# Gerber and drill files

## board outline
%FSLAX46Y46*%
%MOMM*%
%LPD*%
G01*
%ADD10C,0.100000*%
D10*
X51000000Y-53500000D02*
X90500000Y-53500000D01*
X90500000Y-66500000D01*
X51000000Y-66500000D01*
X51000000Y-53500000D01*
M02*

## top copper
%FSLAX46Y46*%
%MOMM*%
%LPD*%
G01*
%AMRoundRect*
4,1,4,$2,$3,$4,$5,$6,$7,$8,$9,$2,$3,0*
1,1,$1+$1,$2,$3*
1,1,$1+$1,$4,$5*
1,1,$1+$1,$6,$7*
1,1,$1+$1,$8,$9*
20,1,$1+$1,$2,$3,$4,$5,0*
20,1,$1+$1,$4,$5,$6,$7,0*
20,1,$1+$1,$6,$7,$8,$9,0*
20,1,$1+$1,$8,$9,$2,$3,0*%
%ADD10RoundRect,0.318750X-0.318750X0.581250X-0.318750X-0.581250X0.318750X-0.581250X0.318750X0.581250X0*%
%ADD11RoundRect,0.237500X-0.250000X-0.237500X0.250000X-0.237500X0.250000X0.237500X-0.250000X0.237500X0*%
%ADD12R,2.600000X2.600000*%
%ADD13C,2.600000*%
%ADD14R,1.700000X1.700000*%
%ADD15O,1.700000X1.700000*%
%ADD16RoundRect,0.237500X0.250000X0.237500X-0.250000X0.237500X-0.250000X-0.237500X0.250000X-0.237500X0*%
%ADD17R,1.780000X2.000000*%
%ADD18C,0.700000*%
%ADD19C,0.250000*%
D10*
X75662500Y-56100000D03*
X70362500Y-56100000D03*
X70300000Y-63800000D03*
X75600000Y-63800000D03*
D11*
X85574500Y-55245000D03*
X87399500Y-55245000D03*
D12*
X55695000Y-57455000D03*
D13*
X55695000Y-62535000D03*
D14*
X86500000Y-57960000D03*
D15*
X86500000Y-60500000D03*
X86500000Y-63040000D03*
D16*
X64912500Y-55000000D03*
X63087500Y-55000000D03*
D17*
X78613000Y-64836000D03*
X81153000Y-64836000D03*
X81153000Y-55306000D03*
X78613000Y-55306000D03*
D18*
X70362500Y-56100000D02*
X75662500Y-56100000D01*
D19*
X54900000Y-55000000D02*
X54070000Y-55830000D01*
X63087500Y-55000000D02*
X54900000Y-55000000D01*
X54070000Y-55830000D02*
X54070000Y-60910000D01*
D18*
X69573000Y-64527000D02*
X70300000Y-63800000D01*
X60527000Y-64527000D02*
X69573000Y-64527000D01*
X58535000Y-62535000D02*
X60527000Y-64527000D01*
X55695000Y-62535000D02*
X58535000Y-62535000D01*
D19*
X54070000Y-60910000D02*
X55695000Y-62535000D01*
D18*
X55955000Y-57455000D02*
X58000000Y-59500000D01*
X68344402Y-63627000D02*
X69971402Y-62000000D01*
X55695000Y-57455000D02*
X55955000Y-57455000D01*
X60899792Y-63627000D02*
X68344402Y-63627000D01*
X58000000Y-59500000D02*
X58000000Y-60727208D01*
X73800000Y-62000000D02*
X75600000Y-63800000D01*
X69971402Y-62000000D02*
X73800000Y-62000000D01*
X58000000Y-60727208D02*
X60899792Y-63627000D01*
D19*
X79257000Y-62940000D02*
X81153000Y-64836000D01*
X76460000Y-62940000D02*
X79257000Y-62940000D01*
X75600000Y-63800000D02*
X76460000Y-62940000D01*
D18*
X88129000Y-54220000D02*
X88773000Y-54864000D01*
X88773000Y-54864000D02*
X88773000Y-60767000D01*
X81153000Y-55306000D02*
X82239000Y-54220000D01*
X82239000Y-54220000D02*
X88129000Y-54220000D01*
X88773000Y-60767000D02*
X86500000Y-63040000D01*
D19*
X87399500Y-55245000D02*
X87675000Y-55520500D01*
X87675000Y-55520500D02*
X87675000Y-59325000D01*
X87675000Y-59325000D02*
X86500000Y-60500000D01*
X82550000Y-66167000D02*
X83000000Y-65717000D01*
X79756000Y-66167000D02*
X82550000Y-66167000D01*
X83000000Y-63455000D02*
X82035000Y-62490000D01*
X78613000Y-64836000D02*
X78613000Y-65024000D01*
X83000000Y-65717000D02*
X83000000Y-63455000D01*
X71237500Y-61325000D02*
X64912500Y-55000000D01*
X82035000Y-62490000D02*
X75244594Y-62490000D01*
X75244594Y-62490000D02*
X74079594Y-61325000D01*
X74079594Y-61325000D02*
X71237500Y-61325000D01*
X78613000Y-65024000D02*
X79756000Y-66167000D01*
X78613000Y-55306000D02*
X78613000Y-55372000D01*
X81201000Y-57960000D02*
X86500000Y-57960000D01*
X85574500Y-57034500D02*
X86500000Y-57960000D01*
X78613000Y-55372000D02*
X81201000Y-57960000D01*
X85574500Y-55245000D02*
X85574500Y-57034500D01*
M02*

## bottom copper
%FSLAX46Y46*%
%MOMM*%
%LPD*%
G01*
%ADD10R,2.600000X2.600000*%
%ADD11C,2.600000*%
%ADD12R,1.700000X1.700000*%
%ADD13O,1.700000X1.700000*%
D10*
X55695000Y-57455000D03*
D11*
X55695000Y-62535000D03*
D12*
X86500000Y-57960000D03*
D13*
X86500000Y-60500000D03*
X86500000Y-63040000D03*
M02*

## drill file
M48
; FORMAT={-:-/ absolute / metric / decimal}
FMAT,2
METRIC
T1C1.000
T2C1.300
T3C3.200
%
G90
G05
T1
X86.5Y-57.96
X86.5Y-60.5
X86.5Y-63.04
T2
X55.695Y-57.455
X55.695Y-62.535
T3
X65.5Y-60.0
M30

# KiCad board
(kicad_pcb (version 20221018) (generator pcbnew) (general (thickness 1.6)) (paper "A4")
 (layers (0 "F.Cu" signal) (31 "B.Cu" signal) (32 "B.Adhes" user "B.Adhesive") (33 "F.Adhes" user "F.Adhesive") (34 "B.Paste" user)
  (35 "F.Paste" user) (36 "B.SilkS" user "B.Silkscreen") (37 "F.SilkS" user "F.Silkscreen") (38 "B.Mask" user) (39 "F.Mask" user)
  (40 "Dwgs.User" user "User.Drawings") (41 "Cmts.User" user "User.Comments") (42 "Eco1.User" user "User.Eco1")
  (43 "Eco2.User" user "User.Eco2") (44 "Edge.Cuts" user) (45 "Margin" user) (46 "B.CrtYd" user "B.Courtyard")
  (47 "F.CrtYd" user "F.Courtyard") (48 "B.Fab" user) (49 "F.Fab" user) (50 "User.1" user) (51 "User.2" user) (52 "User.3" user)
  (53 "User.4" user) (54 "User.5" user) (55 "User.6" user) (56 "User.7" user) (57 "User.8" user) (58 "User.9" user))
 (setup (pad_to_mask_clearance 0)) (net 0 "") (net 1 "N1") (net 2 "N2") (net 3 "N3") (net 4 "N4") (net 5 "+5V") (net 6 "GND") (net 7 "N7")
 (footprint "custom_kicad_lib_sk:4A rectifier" (layer "F.Cu") (at 73 60 -90)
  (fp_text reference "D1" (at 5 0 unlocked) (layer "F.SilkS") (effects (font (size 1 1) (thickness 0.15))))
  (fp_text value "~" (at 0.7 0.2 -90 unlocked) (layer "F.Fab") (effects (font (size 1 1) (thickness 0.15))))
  (pad "1" smd roundrect (at -3.9 -2.6625 270) (size 1.8 1.275) (layers "F.Cu" "F.Paste" "F.Mask") (roundrect_rratio 0.25) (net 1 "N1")
   (thermal_bridge_angle 0))
  (pad "2" smd roundrect (at -3.9 2.6375 270) (size 1.8 1.275) (layers "F.Cu" "F.Paste" "F.Mask") (roundrect_rratio 0.25) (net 1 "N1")
   (thermal_bridge_angle 0))
  (pad "3" smd roundrect (at 3.8 2.7 270) (size 1.8 1.275) (layers "F.Cu" "F.Paste" "F.Mask") (roundrect_rratio 0.25) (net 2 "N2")
   (thermal_bridge_angle 0))
  (pad "4" smd roundrect (at 3.8 -2.6 270) (size 1.8 1.275) (layers "F.Cu" "F.Paste" "F.Mask") (roundrect_rratio 0.25) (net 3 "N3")
   (thermal_bridge_angle 0)))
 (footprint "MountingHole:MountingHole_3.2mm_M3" (layer "F.Cu") (at 65.5 60)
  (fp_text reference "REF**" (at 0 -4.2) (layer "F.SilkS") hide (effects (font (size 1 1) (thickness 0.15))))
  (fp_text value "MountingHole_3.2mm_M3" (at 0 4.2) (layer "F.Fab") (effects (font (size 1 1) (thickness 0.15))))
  (pad "" np_thru_hole circle (at 0 0) (size 3.2 3.2) (drill 3.2) (layers "*.Cu" "*.Mask")))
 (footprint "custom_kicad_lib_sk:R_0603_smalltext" (layer "F.Cu") (at 86.487 55.245)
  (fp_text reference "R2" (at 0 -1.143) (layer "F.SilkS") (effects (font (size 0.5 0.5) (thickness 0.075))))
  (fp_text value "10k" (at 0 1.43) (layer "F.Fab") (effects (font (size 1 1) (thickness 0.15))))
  (pad "1" smd roundrect (at -0.9125 0) (size 0.975 0.95) (layers "F.Cu" "F.Paste" "F.Mask") (roundrect_rratio 0.25) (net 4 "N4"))
  (pad "2" smd roundrect (at 0.9125 0) (size 0.975 0.95) (layers "F.Cu" "F.Paste" "F.Mask") (roundrect_rratio 0.25) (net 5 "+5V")))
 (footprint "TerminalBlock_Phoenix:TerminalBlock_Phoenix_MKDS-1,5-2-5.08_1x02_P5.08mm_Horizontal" (layer "F.Cu") (at 55.695 57.455 -90)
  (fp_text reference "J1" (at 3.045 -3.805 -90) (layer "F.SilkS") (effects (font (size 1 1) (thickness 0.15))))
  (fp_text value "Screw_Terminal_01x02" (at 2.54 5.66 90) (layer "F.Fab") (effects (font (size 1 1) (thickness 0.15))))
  (pad "1" thru_hole rect (at 0 0 270) (size 2.6 2.6) (drill 1.3) (layers "*.Cu" "*.Mask") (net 3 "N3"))
  (pad "2" thru_hole circle (at 5.08 0 270) (size 2.6 2.6) (drill 1.3) (layers "*.Cu" "*.Mask") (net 2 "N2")))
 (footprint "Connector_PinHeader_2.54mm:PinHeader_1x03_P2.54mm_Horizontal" (layer "F.Cu") (at 86.5 57.96)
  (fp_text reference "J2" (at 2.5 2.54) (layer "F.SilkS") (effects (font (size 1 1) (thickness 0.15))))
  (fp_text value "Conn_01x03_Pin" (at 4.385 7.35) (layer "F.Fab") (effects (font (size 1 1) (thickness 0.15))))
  (pad "1" thru_hole rect (at 0 0) (size 1.7 1.7) (drill 1) (layers "*.Cu" "*.Mask") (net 4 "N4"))
  (pad "2" thru_hole oval (at 0 2.54) (size 1.7 1.7) (drill 1) (layers "*.Cu" "*.Mask") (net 5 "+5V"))
  (pad "3" thru_hole oval (at 0 5.08) (size 1.7 1.7) (drill 1) (layers "*.Cu" "*.Mask") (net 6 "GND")))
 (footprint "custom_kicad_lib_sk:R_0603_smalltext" (layer "F.Cu") (at 64 55 180)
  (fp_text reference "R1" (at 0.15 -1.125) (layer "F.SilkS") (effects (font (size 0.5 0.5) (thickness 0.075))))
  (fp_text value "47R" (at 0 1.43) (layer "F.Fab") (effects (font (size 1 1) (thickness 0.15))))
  (pad "1" smd roundrect (at -0.9125 0 180) (size 0.975 0.95) (layers "F.Cu" "F.Paste" "F.Mask") (roundrect_rratio 0.25) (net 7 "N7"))
  (pad "2" smd roundrect (at 0.9125 0 180) (size 0.975 0.95) (layers "F.Cu" "F.Paste" "F.Mask") (roundrect_rratio 0.25) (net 2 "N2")))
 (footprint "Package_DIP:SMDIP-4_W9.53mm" (layer "F.Cu") (at 79.883 60.071 90)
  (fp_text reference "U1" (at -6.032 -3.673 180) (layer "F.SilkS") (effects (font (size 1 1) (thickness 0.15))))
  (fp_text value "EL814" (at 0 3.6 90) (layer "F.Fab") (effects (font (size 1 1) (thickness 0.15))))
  (pad "1" smd rect (at -4.765 -1.27 90) (size 2 1.78) (layers "F.Cu" "F.Paste" "F.Mask") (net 7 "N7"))
  (pad "2" smd rect (at -4.765 1.27 90) (size 2 1.78) (layers "F.Cu" "F.Paste" "F.Mask") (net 3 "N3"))
  (pad "3" smd rect (at 4.765 1.27 90) (size 2 1.78) (layers "F.Cu" "F.Paste" "F.Mask") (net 6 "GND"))
  (pad "4" smd rect (at 4.765 -1.27 90) (size 2 1.78) (layers "F.Cu" "F.Paste" "F.Mask") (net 4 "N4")))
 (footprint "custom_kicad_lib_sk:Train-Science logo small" (layer "B.Cu") (at 74.295 60.325 -90)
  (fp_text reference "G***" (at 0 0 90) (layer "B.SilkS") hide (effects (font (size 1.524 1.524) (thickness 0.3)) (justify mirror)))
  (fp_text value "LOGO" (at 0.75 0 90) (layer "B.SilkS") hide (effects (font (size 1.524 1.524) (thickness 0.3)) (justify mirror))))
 (gr_rect (start 51 53.5) (end 90.5 66.5) (stroke (width 0.1) (type default)) (fill none) (layer "Edge.Cuts"))
 (segment (start 70.3625 56.1) (end 75.6625 56.1) (width 0.7) (layer "F.Cu") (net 1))
 (segment (start 54.9 55) (end 54.07 55.83) (width 0.25) (layer "F.Cu") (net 2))
 (segment (start 63.0875 55) (end 54.9 55) (width 0.25) (layer "F.Cu") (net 2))
 (segment (start 54.07 55.83) (end 54.07 60.91) (width 0.25) (layer "F.Cu") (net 2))
 (segment (start 69.573 64.527) (end 70.3 63.8) (width 0.7) (layer "F.Cu") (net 2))
 (segment (start 60.527 64.527) (end 69.573 64.527) (width 0.7) (layer "F.Cu") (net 2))
 (segment (start 58.535 62.535) (end 60.527 64.527) (width 0.7) (layer "F.Cu") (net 2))
 (segment (start 55.695 62.535) (end 58.535 62.535) (width 0.7) (layer "F.Cu") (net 2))
 (segment (start 54.07 60.91) (end 55.695 62.535) (width 0.25) (layer "F.Cu") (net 2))
 (segment (start 55.955 57.455) (end 58 59.5) (width 0.7) (layer "F.Cu") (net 3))
 (segment (start 68.344402 63.627) (end 69.971402 62) (width 0.7) (layer "F.Cu") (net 3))
 (segment (start 55.695 57.455) (end 55.955 57.455) (width 0.7) (layer "F.Cu") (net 3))
 (segment (start 60.899792 63.627) (end 68.344402 63.627) (width 0.7) (layer "F.Cu") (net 3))
 (segment (start 58 59.5) (end 58 60.727208) (width 0.7) (layer "F.Cu") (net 3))
 (segment (start 73.8 62) (end 75.6 63.8) (width 0.7) (layer "F.Cu") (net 3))
 (segment (start 69.971402 62) (end 73.8 62) (width 0.7) (layer "F.Cu") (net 3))
 (segment (start 58 60.727208) (end 60.899792 63.627) (width 0.7) (layer "F.Cu") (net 3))
 (segment (start 79.257 62.94) (end 81.153 64.836) (width 0.25) (layer "F.Cu") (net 3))
 (segment (start 76.46 62.94) (end 79.257 62.94) (width 0.25) (layer "F.Cu") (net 3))
 (segment (start 75.6 63.8) (end 76.46 62.94) (width 0.25) (layer "F.Cu") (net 3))
 (segment (start 88.129 54.22) (end 88.773 54.864) (width 0.7) (layer "F.Cu") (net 6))
 (segment (start 88.773 54.864) (end 88.773 60.767) (width 0.7) (layer "F.Cu") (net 6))
 (segment (start 81.153 55.306) (end 82.239 54.22) (width 0.7) (layer "F.Cu") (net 6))
 (segment (start 82.239 54.22) (end 88.129 54.22) (width 0.7) (layer "F.Cu") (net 6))
 (segment (start 88.773 60.767) (end 86.5 63.04) (width 0.7) (layer "F.Cu") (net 6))
 (segment (start 87.3995 55.245) (end 87.675 55.5205) (width 0.25) (layer "F.Cu") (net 5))
 (segment (start 87.675 55.5205) (end 87.675 59.325) (width 0.25) (layer "F.Cu") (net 5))
 (segment (start 87.675 59.325) (end 86.5 60.5) (width 0.25) (layer "F.Cu") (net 5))
 (segment (start 82.55 66.167) (end 83 65.717) (width 0.25) (layer "F.Cu") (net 7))
 (segment (start 79.756 66.167) (end 82.55 66.167) (width 0.25) (layer "F.Cu") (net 7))
 (segment (start 83 63.455) (end 82.035 62.49) (width 0.25) (layer "F.Cu") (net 7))
 (segment (start 78.613 64.836) (end 78.613 65.024) (width 0.25) (layer "F.Cu") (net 7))
 (segment (start 83 65.717) (end 83 63.455) (width 0.25) (layer "F.Cu") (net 7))
 (segment (start 71.2375 61.325) (end 64.9125 55) (width 0.25) (layer "F.Cu") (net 7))
 (segment (start 82.035 62.49) (end 75.244594 62.49) (width 0.25) (layer "F.Cu") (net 7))
 (segment (start 75.244594 62.49) (end 74.079594 61.325) (width 0.25) (layer "F.Cu") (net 7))
 (segment (start 74.079594 61.325) (end 71.2375 61.325) (width 0.25) (layer "F.Cu") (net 7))
 (segment (start 78.613 65.024) (end 79.756 66.167) (width 0.25) (layer "F.Cu") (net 7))
 (segment (start 78.613 55.306) (end 78.613 55.372) (width 0.25) (layer "F.Cu") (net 4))
 (segment (start 81.201 57.96) (end 86.5 57.96) (width 0.25) (layer "F.Cu") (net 4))
 (segment (start 85.5745 57.0345) (end 86.5 57.96) (width 0.25) (layer "F.Cu") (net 4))
 (segment (start 78.613 55.372) (end 81.201 57.96) (width 0.25) (layer "F.Cu") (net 4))
 (segment (start 85.5745 55.245) (end 85.5745 57.0345) (width 0.25) (layer "F.Cu") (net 4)))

